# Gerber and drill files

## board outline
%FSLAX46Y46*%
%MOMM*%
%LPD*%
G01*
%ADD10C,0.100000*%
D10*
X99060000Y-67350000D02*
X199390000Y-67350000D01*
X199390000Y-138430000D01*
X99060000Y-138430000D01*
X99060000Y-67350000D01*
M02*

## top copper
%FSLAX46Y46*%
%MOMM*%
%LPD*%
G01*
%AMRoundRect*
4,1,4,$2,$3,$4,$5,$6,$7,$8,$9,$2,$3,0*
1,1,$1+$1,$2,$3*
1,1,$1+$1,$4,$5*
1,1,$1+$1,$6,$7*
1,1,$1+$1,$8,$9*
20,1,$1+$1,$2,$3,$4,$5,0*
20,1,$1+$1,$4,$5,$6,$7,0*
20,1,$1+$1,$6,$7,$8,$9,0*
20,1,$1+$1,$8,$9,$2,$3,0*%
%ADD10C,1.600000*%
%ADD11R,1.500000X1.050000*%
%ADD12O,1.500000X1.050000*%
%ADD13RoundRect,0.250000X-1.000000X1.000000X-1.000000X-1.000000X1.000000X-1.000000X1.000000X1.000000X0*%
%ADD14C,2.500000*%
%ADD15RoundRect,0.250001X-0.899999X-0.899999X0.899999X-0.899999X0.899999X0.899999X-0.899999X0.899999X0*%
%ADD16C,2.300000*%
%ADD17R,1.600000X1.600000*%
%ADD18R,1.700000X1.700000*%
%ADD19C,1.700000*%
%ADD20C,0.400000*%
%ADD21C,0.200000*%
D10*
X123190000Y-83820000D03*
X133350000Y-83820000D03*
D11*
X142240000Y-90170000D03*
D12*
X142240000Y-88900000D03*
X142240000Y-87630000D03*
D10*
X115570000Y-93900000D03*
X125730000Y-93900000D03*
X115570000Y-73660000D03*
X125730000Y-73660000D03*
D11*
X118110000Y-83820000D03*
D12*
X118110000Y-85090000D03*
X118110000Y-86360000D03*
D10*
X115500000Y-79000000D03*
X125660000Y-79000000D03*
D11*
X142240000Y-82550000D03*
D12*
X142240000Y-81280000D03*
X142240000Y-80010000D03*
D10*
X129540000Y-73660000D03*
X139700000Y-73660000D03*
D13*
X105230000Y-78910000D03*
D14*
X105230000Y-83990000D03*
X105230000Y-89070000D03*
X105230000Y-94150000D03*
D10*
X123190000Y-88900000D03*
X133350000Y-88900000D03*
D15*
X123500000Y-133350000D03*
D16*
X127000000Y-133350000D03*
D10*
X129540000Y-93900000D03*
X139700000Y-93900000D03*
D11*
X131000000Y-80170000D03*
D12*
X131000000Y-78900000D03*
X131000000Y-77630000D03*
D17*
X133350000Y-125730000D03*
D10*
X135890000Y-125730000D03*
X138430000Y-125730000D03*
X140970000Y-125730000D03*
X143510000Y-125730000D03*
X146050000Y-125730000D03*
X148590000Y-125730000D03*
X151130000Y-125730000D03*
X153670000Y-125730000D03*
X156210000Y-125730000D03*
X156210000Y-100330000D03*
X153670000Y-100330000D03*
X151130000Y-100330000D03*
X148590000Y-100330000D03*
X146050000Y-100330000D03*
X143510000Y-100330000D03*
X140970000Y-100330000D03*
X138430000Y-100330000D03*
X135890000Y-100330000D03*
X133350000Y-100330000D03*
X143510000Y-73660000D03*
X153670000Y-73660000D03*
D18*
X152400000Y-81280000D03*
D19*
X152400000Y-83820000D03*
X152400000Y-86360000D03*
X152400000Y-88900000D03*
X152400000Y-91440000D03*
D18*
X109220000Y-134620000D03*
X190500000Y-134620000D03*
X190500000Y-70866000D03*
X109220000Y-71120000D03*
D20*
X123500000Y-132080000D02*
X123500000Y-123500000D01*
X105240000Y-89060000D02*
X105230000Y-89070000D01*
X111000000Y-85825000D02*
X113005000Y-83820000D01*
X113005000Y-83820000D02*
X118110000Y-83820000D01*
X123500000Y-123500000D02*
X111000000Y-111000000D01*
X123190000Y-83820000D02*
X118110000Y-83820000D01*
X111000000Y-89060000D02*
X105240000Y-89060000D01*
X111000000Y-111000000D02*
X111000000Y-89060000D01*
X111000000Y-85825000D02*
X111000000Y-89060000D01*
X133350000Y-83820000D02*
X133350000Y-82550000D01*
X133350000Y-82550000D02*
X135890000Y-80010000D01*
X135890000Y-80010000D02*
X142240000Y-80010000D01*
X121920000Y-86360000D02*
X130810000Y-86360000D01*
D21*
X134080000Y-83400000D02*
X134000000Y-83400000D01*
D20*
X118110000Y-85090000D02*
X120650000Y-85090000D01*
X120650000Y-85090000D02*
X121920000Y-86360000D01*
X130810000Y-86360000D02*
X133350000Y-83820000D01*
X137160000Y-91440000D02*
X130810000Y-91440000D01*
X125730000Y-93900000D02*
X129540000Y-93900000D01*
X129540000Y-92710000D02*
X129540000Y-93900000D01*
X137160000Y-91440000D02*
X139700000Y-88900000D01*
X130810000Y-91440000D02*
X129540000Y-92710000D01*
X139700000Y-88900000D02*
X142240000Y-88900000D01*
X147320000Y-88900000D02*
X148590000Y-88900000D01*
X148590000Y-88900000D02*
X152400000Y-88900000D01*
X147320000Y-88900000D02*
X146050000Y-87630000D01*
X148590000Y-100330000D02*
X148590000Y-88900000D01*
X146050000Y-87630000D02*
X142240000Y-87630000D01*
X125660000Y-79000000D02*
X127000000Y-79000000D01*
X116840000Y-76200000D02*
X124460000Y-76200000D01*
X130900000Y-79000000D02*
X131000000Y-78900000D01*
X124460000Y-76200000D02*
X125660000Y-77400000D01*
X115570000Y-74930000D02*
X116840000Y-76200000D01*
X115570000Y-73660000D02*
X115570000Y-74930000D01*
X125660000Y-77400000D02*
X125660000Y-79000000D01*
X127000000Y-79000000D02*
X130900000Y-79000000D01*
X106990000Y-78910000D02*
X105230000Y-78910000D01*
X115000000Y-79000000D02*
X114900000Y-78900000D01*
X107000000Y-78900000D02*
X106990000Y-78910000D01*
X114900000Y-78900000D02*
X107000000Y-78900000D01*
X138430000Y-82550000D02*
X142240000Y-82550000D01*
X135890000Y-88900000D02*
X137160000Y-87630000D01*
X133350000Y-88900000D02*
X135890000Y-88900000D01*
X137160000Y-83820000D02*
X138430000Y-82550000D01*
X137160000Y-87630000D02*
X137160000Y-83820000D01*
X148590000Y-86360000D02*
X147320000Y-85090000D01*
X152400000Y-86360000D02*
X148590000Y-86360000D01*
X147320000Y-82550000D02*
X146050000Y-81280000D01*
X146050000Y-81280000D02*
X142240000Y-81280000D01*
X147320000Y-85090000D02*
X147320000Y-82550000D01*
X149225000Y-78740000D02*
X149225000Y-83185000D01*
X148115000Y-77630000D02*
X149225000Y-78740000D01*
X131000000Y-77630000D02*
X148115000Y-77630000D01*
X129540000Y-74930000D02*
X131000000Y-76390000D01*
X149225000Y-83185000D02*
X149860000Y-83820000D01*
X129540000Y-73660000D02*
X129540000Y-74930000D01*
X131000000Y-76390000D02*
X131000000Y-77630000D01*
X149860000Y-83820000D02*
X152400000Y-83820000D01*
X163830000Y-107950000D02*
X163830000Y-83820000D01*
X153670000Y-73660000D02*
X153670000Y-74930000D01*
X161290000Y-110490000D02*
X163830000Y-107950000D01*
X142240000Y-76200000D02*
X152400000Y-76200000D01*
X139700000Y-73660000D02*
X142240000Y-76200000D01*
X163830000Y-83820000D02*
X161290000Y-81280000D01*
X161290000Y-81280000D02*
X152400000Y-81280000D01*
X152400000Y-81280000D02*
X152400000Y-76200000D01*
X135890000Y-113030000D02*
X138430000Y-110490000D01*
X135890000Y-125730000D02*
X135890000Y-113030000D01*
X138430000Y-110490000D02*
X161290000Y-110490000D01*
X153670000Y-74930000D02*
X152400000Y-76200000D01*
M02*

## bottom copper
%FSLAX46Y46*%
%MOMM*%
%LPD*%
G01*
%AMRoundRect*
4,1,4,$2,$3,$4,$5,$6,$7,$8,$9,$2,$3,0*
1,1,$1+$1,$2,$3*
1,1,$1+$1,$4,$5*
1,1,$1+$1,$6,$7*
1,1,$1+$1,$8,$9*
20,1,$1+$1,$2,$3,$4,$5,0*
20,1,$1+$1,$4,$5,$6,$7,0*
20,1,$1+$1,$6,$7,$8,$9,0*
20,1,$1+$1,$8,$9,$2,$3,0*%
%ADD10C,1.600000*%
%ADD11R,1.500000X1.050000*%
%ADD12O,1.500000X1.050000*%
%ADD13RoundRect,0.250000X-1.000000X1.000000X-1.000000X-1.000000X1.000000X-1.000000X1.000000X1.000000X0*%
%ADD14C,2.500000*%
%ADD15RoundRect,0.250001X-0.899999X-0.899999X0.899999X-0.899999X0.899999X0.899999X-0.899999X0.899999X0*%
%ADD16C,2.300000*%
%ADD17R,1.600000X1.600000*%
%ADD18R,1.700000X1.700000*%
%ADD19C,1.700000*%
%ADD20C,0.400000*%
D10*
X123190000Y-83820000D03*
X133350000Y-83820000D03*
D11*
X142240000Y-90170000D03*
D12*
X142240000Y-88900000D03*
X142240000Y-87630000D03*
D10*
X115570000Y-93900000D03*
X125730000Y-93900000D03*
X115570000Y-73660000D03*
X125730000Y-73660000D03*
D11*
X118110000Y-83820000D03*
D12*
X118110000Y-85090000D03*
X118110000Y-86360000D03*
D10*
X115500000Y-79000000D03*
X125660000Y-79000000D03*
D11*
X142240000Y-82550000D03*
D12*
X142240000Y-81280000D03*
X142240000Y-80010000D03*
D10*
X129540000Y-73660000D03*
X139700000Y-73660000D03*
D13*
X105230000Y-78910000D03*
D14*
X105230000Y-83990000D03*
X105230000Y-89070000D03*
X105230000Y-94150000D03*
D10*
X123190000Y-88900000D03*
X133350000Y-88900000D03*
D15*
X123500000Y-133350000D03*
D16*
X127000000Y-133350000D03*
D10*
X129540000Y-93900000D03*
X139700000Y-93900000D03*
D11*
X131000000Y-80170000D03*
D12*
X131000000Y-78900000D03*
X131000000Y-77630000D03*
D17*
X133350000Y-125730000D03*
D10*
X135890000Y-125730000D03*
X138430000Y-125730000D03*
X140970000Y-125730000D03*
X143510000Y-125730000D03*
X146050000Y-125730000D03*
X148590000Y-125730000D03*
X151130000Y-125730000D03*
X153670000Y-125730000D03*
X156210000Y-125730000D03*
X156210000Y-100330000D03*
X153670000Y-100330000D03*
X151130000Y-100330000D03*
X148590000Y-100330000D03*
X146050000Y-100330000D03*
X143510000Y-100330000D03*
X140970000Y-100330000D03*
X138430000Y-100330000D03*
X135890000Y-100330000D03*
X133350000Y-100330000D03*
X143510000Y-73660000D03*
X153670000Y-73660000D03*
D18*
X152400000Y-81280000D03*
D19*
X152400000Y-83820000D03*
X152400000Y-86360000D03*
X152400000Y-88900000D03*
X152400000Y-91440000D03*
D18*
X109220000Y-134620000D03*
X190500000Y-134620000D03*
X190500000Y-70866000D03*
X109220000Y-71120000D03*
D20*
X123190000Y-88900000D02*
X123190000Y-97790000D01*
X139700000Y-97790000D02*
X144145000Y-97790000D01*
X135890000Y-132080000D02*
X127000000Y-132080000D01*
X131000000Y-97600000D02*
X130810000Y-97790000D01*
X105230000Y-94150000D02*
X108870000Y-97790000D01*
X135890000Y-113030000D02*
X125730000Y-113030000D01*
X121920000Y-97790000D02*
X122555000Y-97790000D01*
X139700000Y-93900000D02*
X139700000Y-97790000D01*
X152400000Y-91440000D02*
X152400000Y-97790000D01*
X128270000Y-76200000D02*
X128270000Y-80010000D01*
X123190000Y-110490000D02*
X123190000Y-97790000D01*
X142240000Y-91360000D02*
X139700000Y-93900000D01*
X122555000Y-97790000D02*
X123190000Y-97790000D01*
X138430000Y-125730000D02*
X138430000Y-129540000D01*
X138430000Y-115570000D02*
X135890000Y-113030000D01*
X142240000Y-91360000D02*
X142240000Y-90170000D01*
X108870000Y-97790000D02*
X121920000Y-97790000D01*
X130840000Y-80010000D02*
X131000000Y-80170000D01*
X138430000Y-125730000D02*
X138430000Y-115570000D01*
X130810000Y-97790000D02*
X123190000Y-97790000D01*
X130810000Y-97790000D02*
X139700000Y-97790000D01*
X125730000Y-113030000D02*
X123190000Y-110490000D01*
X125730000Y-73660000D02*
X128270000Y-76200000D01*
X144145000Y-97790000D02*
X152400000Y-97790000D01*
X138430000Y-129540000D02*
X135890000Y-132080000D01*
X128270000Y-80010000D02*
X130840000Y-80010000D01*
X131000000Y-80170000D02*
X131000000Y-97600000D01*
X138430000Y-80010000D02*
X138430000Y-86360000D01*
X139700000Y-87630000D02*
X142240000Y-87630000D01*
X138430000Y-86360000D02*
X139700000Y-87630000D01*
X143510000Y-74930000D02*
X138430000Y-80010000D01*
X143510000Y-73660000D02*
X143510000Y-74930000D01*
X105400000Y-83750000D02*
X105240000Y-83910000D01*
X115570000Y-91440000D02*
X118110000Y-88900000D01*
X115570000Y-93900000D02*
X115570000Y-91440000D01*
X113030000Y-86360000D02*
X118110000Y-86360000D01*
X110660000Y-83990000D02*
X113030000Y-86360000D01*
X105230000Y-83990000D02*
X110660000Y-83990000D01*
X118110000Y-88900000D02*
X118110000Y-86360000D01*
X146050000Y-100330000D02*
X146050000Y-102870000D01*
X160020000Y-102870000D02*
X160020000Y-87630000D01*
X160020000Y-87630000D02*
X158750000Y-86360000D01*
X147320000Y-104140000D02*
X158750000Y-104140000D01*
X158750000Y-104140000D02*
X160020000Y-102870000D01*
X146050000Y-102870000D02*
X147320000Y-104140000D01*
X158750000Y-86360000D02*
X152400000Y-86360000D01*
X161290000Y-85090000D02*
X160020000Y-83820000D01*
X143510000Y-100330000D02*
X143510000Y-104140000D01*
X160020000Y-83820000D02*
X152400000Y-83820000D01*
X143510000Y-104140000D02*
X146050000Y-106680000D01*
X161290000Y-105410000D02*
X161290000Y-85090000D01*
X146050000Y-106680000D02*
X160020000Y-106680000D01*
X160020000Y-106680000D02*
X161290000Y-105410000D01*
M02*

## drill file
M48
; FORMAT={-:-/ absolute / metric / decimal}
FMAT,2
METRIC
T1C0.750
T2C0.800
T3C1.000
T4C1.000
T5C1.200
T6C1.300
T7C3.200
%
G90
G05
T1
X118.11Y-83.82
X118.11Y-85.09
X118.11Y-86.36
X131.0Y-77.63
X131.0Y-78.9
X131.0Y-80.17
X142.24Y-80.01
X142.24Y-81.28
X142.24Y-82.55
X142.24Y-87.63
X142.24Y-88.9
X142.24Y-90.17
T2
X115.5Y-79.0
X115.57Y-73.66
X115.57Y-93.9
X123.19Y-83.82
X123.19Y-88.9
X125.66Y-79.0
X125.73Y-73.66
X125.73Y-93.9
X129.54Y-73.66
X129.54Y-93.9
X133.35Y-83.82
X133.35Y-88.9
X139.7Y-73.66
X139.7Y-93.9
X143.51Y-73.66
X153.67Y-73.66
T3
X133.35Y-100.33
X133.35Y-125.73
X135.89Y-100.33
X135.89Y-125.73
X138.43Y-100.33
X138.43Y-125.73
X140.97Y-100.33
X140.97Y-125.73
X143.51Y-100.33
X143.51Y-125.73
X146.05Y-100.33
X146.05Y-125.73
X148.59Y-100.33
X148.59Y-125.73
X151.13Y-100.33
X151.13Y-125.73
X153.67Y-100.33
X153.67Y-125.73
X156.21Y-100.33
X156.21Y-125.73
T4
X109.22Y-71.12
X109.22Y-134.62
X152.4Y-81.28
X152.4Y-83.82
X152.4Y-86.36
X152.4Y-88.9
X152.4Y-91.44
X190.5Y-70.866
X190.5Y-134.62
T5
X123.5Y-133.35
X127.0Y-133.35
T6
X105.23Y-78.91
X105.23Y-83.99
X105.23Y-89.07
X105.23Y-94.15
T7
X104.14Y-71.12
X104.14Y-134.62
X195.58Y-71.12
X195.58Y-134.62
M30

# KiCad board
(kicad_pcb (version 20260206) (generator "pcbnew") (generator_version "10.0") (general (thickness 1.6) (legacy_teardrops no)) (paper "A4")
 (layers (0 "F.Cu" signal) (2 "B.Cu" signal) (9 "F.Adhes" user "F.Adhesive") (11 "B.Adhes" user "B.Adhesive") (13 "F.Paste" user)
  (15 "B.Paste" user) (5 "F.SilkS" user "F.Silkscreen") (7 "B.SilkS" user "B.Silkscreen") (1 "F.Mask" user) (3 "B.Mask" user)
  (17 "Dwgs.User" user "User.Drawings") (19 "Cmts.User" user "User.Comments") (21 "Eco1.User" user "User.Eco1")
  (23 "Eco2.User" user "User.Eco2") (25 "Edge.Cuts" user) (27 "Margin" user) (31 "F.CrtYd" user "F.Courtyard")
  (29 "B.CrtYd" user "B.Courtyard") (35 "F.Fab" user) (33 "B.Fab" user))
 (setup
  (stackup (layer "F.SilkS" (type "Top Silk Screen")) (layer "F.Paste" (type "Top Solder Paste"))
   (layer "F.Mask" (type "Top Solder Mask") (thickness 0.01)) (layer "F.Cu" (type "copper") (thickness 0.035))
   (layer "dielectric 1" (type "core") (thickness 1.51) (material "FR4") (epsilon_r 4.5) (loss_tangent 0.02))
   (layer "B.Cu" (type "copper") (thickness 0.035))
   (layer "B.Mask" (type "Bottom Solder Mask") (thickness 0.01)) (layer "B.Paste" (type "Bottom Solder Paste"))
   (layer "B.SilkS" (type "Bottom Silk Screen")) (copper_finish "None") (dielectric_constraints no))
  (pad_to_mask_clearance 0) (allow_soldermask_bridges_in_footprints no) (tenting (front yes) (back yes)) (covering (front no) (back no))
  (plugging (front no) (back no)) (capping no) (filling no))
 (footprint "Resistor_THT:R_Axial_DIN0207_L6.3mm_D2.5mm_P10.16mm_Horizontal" (layer "F.Cu") (at 123.19 83.82)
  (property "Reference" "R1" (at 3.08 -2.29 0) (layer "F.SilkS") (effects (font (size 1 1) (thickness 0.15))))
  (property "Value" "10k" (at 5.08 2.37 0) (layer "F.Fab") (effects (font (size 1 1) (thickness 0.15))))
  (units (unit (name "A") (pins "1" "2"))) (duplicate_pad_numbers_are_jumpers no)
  (pad "1" thru_hole circle (at 0 0) (size 1.6 1.6) (drill 0.8) (layers "*.Cu" "*.Mask") (remove_unused_layers no) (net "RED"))
  (pad "2" thru_hole circle (at 10.16 0) (size 1.6 1.6) (drill 0.8) (layers "*.Cu" "*.Mask") (remove_unused_layers no) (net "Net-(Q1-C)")))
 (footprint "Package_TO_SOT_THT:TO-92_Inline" (layer "F.Cu") (at 142.24 90.17 90)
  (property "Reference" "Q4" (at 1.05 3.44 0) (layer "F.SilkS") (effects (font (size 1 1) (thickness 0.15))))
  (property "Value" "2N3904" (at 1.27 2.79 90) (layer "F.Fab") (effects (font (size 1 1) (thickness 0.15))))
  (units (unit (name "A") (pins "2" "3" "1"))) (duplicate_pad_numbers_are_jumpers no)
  (pad "1" thru_hole rect (at 0 0 90) (size 1.05 1.5) (drill 0.75) (layers "*.Cu" "*.Mask") (remove_unused_layers no) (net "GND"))
  (pad "2" thru_hole oval (at 1.27 0 90) (size 1.05 1.5) (drill 0.75) (layers "*.Cu" "*.Mask") (remove_unused_layers no) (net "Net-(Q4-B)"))
  (pad "3" thru_hole oval (at 2.54 0 90) (size 1.05 1.5) (drill 0.75) (layers "*.Cu" "*.Mask") (remove_unused_layers no) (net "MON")))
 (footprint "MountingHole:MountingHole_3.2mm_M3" (layer "F.Cu") (at 195.58 134.62)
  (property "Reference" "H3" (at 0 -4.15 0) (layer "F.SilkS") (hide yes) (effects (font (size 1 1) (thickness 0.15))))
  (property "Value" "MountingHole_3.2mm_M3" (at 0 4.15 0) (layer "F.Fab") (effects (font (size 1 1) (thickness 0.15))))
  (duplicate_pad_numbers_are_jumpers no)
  (pad "" np_thru_hole circle (at 0 0) (size 3.2 3.2) (drill 3.2) (layers "*.Cu" "*.Mask")))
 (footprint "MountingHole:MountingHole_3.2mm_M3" (layer "F.Cu") (at 104.14 71.12)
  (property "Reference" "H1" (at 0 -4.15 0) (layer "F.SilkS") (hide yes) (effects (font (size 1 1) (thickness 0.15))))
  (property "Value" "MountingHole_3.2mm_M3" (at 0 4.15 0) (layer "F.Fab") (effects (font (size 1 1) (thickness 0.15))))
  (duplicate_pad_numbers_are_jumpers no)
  (pad "" np_thru_hole circle (at 0 0) (size 3.2 3.2) (drill 3.2) (layers "*.Cu" "*.Mask")))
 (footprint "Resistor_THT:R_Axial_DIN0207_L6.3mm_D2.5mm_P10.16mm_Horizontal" (layer "F.Cu") (at 115.57 93.9)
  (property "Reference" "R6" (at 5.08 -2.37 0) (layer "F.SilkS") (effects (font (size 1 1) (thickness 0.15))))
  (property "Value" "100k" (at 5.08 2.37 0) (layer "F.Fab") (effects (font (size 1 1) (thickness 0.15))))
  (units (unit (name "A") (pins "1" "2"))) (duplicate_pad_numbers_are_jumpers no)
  (pad "1" thru_hole circle (at 0 0) (size 1.6 1.6) (drill 0.8) (layers "*.Cu" "*.Mask") (remove_unused_layers no) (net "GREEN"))
  (pad "2" thru_hole circle (at 10.16 0) (size 1.6 1.6) (drill 0.8) (layers "*.Cu" "*.Mask") (remove_unused_layers no) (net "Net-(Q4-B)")))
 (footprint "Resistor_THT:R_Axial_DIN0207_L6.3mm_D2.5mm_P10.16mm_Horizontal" (layer "F.Cu") (at 115.57 73.66)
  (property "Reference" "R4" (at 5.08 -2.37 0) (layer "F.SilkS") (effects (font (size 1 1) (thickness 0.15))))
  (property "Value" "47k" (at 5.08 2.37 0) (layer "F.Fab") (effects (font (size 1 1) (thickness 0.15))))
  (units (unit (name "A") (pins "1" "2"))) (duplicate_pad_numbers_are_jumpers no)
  (pad "1" thru_hole circle (at 0 0) (size 1.6 1.6) (drill 0.8) (layers "*.Cu" "*.Mask") (remove_unused_layers no) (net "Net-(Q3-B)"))
  (pad "2" thru_hole circle (at 10.16 0) (size 1.6 1.6) (drill 0.8) (layers "*.Cu" "*.Mask") (remove_unused_layers no) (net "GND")))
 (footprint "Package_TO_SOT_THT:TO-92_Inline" (layer "F.Cu") (at 118.11 83.82 -90)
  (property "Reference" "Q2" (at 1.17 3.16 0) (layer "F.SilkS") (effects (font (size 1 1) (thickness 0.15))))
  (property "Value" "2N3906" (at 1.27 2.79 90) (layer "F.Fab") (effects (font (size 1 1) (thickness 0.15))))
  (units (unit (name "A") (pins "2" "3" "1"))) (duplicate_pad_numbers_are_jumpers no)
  (pad "1" thru_hole rect (at 0 0 270) (size 1.05 1.5) (drill 0.75) (layers "*.Cu" "*.Mask") (remove_unused_layers no) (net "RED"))
  (pad "2" thru_hole oval (at 1.27 0 270) (size 1.05 1.5) (drill 0.75) (layers "*.Cu" "*.Mask") (remove_unused_layers no) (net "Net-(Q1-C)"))
  (pad "3" thru_hole oval (at 2.54 0 270) (size 1.05 1.5) (drill 0.75) (layers "*.Cu" "*.Mask") (remove_unused_layers no) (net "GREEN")))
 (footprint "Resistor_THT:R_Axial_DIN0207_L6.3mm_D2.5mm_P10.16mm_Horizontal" (layer "F.Cu") (at 115.5 79)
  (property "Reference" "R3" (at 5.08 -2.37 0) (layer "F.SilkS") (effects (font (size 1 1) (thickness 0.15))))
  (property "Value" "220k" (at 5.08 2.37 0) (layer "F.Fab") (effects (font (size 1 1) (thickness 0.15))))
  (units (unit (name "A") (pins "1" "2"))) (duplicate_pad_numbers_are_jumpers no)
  (pad "1" thru_hole circle (at 0 0) (size 1.6 1.6) (drill 0.8) (layers "*.Cu" "*.Mask") (remove_unused_layers no) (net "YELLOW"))
  (pad "2" thru_hole circle (at 10.16 0) (size 1.6 1.6) (drill 0.8) (layers "*.Cu" "*.Mask") (remove_unused_layers no) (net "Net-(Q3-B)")))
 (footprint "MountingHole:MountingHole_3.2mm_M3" (layer "F.Cu") (at 195.58 71.12)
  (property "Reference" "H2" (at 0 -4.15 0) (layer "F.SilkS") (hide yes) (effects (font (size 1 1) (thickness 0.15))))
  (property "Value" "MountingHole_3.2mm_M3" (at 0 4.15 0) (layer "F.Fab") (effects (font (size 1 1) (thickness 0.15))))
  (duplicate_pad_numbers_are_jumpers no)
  (pad "" np_thru_hole circle (at 0 0) (size 3.2 3.2) (drill 3.2) (layers "*.Cu" "*.Mask")))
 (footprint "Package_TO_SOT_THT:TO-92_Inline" (layer "F.Cu") (at 142.24 82.55 90)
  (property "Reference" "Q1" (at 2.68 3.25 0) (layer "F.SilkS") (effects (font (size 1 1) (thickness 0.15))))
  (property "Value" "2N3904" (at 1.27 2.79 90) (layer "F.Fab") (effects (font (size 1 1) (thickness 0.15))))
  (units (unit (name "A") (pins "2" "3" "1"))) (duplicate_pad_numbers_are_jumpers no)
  (pad "1" thru_hole rect (at 0 0 90) (size 1.05 1.5) (drill 0.75) (layers "*.Cu" "*.Mask") (remove_unused_layers no) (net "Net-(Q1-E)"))
  (pad "2" thru_hole oval (at 1.27 0 90) (size 1.05 1.5) (drill 0.75) (layers "*.Cu" "*.Mask") (remove_unused_layers no) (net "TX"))
  (pad "3" thru_hole oval (at 2.54 0 90) (size 1.05 1.5) (drill 0.75) (layers "*.Cu" "*.Mask") (remove_unused_layers no) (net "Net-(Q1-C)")))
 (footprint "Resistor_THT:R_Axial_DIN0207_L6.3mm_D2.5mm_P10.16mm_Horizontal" (layer "F.Cu") (at 129.54 73.66)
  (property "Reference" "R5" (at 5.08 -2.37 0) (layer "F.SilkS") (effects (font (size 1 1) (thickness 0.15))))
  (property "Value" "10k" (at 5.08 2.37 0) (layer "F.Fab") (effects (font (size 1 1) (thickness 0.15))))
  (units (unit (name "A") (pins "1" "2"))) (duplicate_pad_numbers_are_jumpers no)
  (pad "1" thru_hole circle (at 0 0) (size 1.6 1.6) (drill 0.8) (layers "*.Cu" "*.Mask") (remove_unused_layers no) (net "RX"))
  (pad "2" thru_hole circle (at 10.16 0) (size 1.6 1.6) (drill 0.8) (layers "*.Cu" "*.Mask") (remove_unused_layers no) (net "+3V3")))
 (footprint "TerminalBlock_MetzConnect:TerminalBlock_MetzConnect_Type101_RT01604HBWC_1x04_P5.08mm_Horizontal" (layer "F.Cu")
  (at 105.23 78.91 -90)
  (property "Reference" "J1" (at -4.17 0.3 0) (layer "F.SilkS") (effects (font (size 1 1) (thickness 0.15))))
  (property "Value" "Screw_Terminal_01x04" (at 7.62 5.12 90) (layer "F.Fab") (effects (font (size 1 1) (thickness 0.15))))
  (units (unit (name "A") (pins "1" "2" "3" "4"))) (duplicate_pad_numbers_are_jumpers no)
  (pad "1" thru_hole roundrect (at 0 0 270) (size 2.5 2.5) (drill 1.3) (layers "*.Cu" "*.Mask") (remove_unused_layers no)
   (roundrect_rratio 0.1) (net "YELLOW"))
  (pad "2" thru_hole circle (at 5.08 0 270) (size 2.5 2.5) (drill 1.3) (layers "*.Cu" "*.Mask") (remove_unused_layers no) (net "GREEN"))
  (pad "3" thru_hole circle (at 10.16 0 270) (size 2.5 2.5) (drill 1.3) (layers "*.Cu" "*.Mask") (remove_unused_layers no) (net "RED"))
  (pad "4" thru_hole circle (at 15.24 0 270) (size 2.5 2.5) (drill 1.3) (layers "*.Cu" "*.Mask") (remove_unused_layers no) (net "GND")))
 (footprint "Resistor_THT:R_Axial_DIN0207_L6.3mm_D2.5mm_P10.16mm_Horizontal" (layer "F.Cu") (at 123.19 88.9)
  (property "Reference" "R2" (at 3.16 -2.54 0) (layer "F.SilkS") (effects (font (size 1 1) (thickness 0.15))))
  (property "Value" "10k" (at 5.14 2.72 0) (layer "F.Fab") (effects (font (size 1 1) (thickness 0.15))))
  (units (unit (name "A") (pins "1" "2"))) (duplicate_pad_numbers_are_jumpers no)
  (pad "1" thru_hole circle (at 0 0) (size 1.6 1.6) (drill 0.8) (layers "*.Cu" "*.Mask") (remove_unused_layers no) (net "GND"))
  (pad "2" thru_hole circle (at 10.16 0) (size 1.6 1.6) (drill 0.8) (layers "*.Cu" "*.Mask") (remove_unused_layers no) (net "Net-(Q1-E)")))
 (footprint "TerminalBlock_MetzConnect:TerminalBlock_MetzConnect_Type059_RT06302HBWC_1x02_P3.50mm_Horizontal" (layer "F.Cu")
  (at 123.5 133.35)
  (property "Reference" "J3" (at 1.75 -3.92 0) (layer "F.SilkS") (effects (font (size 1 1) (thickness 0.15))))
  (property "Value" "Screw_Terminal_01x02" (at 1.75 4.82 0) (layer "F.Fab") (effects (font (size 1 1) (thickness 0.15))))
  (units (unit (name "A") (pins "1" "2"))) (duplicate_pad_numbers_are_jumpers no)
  (pad "1" thru_hole roundrect (at 0 0) (size 2.3 2.3) (drill 1.2) (layers "*.Cu" "*.Mask") (remove_unused_layers no)
   (roundrect_rratio 0.108696) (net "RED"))
  (pad "2" thru_hole circle (at 3.5 0) (size 2.3 2.3) (drill 1.2) (layers "*.Cu" "*.Mask") (remove_unused_layers no) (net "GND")))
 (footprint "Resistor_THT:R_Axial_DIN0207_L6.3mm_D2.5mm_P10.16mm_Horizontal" (layer "F.Cu") (at 129.54 93.9)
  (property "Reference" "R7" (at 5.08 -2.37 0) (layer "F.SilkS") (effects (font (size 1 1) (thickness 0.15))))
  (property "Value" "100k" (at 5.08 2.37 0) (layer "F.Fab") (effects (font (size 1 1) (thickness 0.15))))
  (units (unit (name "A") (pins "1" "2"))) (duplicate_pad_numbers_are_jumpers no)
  (pad "1" thru_hole circle (at 0 0) (size 1.6 1.6) (drill 0.8) (layers "*.Cu" "*.Mask") (remove_unused_layers no) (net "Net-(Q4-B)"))
  (pad "2" thru_hole circle (at 10.16 0) (size 1.6 1.6) (drill 0.8) (layers "*.Cu" "*.Mask") (remove_unused_layers no) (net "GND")))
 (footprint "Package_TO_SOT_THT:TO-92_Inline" (layer "F.Cu") (at 131 80.17 90)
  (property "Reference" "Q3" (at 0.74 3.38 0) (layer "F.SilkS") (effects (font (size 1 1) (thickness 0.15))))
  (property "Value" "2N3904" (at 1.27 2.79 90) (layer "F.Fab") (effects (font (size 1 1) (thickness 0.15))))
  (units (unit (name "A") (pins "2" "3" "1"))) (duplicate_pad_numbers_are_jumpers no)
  (pad "1" thru_hole rect (at 0 0 90) (size 1.05 1.5) (drill 0.75) (layers "*.Cu" "*.Mask") (remove_unused_layers no) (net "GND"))
  (pad "2" thru_hole oval (at 1.27 0 90) (size 1.05 1.5) (drill 0.75) (layers "*.Cu" "*.Mask") (remove_unused_layers no) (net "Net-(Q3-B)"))
  (pad "3" thru_hole oval (at 2.54 0 90) (size 1.05 1.5) (drill 0.75) (layers "*.Cu" "*.Mask") (remove_unused_layers no) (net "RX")))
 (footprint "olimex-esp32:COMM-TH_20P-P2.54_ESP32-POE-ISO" (layer "F.Cu") (at 144.78 113.03 90)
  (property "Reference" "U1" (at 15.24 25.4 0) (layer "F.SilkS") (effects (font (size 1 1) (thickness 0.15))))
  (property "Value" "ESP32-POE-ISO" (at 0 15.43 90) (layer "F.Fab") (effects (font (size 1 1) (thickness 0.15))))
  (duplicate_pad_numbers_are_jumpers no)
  (pad "1" thru_hole rect (at -12.7 -11.43 90) (size 1.6 1.6) (drill 0.999998) (layers "*.Cu" "*.Mask") (remove_unused_layers no)
   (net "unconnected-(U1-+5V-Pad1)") (thermal_bridge_angle 45))
  (pad "2" thru_hole circle (at -12.7 -8.89 90) (size 1.6 1.6) (drill 0.999998) (layers "*.Cu" "*.Mask") (remove_unused_layers no)
   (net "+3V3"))
  (pad "3" thru_hole circle (at -12.7 -6.35 90) (size 1.6 1.6) (drill 0.999998) (layers "*.Cu" "*.Mask") (remove_unused_layers no)
   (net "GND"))
  (pad "4" thru_hole circle (at -12.7 -3.81 90) (size 1.6 1.6) (drill 0.999998) (layers "*.Cu" "*.Mask") (remove_unused_layers no)
   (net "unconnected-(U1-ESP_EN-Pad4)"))
  (pad "5" thru_hole circle (at -12.7 -1.27 90) (size 1.6 1.6) (drill 0.999998) (layers "*.Cu" "*.Mask") (remove_unused_layers no)
   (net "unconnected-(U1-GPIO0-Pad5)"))
  (pad "6" thru_hole circle (at -12.7 1.27 90) (size 1.6 1.6) (drill 0.999998) (layers "*.Cu" "*.Mask") (remove_unused_layers no)
   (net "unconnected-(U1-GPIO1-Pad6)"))
  (pad "7" thru_hole circle (at -12.7 3.81 90) (size 1.6 1.6) (drill 0.999998) (layers "*.Cu" "*.Mask") (remove_unused_layers no)
   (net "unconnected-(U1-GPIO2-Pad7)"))
  (pad "8" thru_hole circle (at -12.7 6.35 90) (size 1.6 1.6) (drill 0.999998) (layers "*.Cu" "*.Mask") (remove_unused_layers no)
   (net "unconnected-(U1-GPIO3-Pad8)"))
  (pad "9" thru_hole circle (at -12.7 8.89 90) (size 1.6 1.6) (drill 0.999998) (layers "*.Cu" "*.Mask") (remove_unused_layers no)
   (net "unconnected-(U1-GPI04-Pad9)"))
  (pad "10" thru_hole circle (at -12.7 11.43 90) (size 1.6 1.6) (drill 0.999998) (layers "*.Cu" "*.Mask") (remove_unused_layers no)
   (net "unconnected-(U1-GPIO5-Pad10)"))
  (pad "11" thru_hole circle (at 12.7 11.43 90) (size 1.6 1.6) (drill 0.999998) (layers "*.Cu" "*.Mask") (remove_unused_layers no)
   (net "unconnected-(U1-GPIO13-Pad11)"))
  (pad "12" thru_hole circle (at 12.7 8.89 90) (size 1.6 1.6) (drill 0.999998) (layers "*.Cu" "*.Mask") (remove_unused_layers no)
   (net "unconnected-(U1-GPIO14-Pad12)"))
  (pad "13" thru_hole circle (at 12.7 6.35 90) (size 1.6 1.6) (drill 0.999998) (layers "*.Cu" "*.Mask") (remove_unused_layers no)
   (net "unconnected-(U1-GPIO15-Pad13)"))
  (pad "14" thru_hole circle (at 12.7 3.81 90) (size 1.6 1.6) (drill 0.999998) (layers "*.Cu" "*.Mask") (remove_unused_layers no)
   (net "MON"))
  (pad "15" thru_hole circle (at 12.7 1.27 90) (size 1.6 1.6) (drill 0.999998) (layers "*.Cu" "*.Mask") (remove_unused_layers no) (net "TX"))
  (pad "16" thru_hole circle (at 12.7 -1.27 90) (size 1.6 1.6) (drill 0.999998) (layers "*.Cu" "*.Mask") (remove_unused_layers no)
   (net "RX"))
  (pad "17" thru_hole circle (at 12.7 -3.81 90) (size 1.6 1.6) (drill 0.999998) (layers "*.Cu" "*.Mask") (remove_unused_layers no)
   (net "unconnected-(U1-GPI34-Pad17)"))
  (pad "18" thru_hole circle (at 12.7 -6.35 90) (size 1.6 1.6) (drill 0.999998) (layers "*.Cu" "*.Mask") (remove_unused_layers no)
   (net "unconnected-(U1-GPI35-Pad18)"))
  (pad "19" thru_hole circle (at 12.7 -8.89 90) (size 1.6 1.6) (drill 0.999998) (layers "*.Cu" "*.Mask") (remove_unused_layers no)
   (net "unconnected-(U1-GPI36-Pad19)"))
  (pad "20" thru_hole circle (at 12.7 -11.43 90) (size 1.6 1.6) (drill 0.999998) (layers "*.Cu" "*.Mask") (remove_unused_layers no)
   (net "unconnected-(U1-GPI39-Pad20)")))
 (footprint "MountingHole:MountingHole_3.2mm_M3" (layer "F.Cu") (at 104.14 134.62)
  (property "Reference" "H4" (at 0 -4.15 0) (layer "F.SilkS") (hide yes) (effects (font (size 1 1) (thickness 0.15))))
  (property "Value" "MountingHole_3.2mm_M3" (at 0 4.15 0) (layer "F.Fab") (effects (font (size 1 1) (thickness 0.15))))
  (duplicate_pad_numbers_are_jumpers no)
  (pad "" np_thru_hole circle (at 0 0) (size 3.2 3.2) (drill 3.2) (layers "*.Cu" "*.Mask")))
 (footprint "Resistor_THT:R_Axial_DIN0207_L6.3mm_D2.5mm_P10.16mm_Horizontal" (layer "F.Cu") (at 143.51 73.66)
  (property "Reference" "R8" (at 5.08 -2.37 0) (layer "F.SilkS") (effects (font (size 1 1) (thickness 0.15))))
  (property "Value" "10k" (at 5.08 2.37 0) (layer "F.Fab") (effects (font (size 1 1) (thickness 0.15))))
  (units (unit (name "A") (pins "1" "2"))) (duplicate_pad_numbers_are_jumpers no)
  (pad "1" thru_hole circle (at 0 0) (size 1.6 1.6) (drill 0.8) (layers "*.Cu" "*.Mask") (remove_unused_layers no) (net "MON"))
  (pad "2" thru_hole circle (at 10.16 0) (size 1.6 1.6) (drill 0.8) (layers "*.Cu" "*.Mask") (remove_unused_layers no) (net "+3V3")))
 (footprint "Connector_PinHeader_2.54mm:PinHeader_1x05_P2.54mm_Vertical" (layer "F.Cu") (at 152.4 81.28)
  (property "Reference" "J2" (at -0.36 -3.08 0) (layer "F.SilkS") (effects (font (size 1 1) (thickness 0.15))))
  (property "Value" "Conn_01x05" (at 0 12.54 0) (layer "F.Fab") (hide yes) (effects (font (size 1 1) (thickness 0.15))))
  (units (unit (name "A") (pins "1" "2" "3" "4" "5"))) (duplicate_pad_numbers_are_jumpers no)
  (pad "1" thru_hole rect (at 0 0) (size 1.7 1.7) (drill 1) (layers "*.Cu" "*.Mask") (remove_unused_layers no) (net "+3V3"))
  (pad "2" thru_hole circle (at 0 2.54) (size 1.7 1.7) (drill 1) (layers "*.Cu" "*.Mask") (remove_unused_layers no) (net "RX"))
  (pad "3" thru_hole circle (at 0 5.08) (size 1.7 1.7) (drill 1) (layers "*.Cu" "*.Mask") (remove_unused_layers no) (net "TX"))
  (pad "4" thru_hole circle (at 0 7.62) (size 1.7 1.7) (drill 1) (layers "*.Cu" "*.Mask") (remove_unused_layers no) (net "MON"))
  (pad "5" thru_hole circle (at 0 10.16) (size 1.7 1.7) (drill 1) (layers "*.Cu" "*.Mask") (remove_unused_layers no) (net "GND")))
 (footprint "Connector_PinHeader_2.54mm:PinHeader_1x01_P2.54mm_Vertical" (layer "B.Cu") (at 109.22 134.62)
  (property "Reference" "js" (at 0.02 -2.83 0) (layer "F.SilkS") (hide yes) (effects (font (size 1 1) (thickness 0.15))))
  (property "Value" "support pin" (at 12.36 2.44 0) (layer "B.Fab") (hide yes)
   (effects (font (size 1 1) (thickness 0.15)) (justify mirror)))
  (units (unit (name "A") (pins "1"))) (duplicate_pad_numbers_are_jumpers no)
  (pad "1" thru_hole rect (at 0 0) (size 1.7 1.7) (drill 1) (layers "*.Cu" "*.Mask") (remove_unused_layers no)
   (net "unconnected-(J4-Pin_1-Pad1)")))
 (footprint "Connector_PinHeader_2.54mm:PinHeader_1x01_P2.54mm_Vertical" (layer "B.Cu") (at 190.5 134.62)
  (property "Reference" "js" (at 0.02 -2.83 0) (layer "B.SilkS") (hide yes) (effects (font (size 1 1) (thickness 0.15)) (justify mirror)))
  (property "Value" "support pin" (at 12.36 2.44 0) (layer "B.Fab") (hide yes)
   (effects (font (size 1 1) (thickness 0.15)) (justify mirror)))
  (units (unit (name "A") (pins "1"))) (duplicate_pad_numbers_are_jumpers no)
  (pad "1" thru_hole rect (at 0 0) (size 1.7 1.7) (drill 1) (layers "*.Cu" "*.Mask") (remove_unused_layers no)
   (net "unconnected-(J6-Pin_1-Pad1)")))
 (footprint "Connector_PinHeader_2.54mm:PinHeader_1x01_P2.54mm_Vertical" (layer "B.Cu") (at 190.5 70.866)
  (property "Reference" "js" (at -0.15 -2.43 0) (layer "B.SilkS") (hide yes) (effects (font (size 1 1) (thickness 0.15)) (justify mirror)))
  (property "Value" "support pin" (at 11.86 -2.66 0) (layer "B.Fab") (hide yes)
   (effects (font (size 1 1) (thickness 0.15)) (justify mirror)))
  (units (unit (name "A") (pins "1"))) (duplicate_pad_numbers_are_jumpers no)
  (pad "1" thru_hole rect (at 0 0) (size 1.7 1.7) (drill 1) (layers "*.Cu" "*.Mask") (remove_unused_layers no)
   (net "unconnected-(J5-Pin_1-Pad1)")))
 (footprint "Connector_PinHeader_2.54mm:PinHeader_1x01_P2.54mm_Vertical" (layer "B.Cu") (at 109.22 71.12)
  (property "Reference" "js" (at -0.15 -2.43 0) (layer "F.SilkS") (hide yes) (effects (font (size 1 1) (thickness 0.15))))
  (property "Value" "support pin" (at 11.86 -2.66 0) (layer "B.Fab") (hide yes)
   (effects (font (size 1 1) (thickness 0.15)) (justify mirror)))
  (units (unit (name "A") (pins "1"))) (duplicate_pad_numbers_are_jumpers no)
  (pad "1" thru_hole rect (at 0 0) (size 1.7 1.7) (drill 1) (layers "*.Cu" "*.Mask") (remove_unused_layers no)
   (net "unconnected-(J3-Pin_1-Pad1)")))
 (gr_rect (start 99.06 67.35) (end 199.39 138.43) (stroke (width 0.1) (type default)) (fill no) (layer "Edge.Cuts"))
 (segment (start 123.5 132.08) (end 123.5 123.5) (width 0.4) (layer "F.Cu") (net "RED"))
 (segment (start 105.24 89.06) (end 105.23 89.07) (width 0.4) (layer "F.Cu") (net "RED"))
 (segment (start 111 85.825) (end 113.005 83.82) (width 0.4) (layer "F.Cu") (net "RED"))
 (segment (start 113.005 83.82) (end 118.11 83.82) (width 0.4) (layer "F.Cu") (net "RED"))
 (segment (start 123.5 123.5) (end 111 111) (width 0.4) (layer "F.Cu") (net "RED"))
 (segment (start 123.19 83.82) (end 118.11 83.82) (width 0.4) (layer "F.Cu") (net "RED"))
 (segment (start 111 89.06) (end 105.24 89.06) (width 0.4) (layer "F.Cu") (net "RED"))
 (segment (start 111 111) (end 111 89.06) (width 0.4) (layer "F.Cu") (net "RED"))
 (segment (start 111 85.825) (end 111 89.06) (width 0.4) (layer "F.Cu") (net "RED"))
 (segment (start 133.35 83.82) (end 133.35 82.55) (width 0.4) (layer "F.Cu") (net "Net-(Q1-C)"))
 (segment (start 133.35 82.55) (end 135.89 80.01) (width 0.4) (layer "F.Cu") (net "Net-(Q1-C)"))
 (segment (start 135.89 80.01) (end 142.24 80.01) (width 0.4) (layer "F.Cu") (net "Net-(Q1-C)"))
 (segment (start 121.92 86.36) (end 130.81 86.36) (width 0.4) (layer "F.Cu") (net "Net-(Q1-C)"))
 (segment (start 134.08 83.4) (end 134 83.4) (width 0.2) (layer "F.Cu") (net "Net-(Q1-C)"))
 (segment (start 118.11 85.09) (end 120.65 85.09) (width 0.4) (layer "F.Cu") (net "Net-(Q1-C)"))
 (segment (start 120.65 85.09) (end 121.92 86.36) (width 0.4) (layer "F.Cu") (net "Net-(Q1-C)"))
 (segment (start 130.81 86.36) (end 133.35 83.82) (width 0.4) (layer "F.Cu") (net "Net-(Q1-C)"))
 (segment (start 123.19 88.9) (end 123.19 97.79) (width 0.4) (layer "B.Cu") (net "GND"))
 (segment (start 139.7 97.79) (end 144.145 97.79) (width 0.4) (layer "B.Cu") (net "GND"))
 (segment (start 135.89 132.08) (end 127 132.08) (width 0.4) (layer "B.Cu") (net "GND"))
 (segment (start 131 97.6) (end 130.81 97.79) (width 0.4) (layer "B.Cu") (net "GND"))
 (segment (start 105.23 94.15) (end 108.87 97.79) (width 0.4) (layer "B.Cu") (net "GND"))
 (segment (start 135.89 113.03) (end 125.73 113.03) (width 0.4) (layer "B.Cu") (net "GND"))
 (segment (start 121.92 97.79) (end 122.555 97.79) (width 0.4) (layer "B.Cu") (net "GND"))
 (segment (start 139.7 93.9) (end 139.7 97.79) (width 0.4) (layer "B.Cu") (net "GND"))
 (segment (start 152.4 91.44) (end 152.4 97.79) (width 0.4) (layer "B.Cu") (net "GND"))
 (segment (start 128.27 76.2) (end 128.27 80.01) (width 0.4) (layer "B.Cu") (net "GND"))
 (segment (start 123.19 110.49) (end 123.19 97.79) (width 0.4) (layer "B.Cu") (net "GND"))
 (segment (start 142.24 91.36) (end 139.7 93.9) (width 0.4) (layer "B.Cu") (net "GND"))
 (segment (start 122.555 97.79) (end 123.19 97.79) (width 0.4) (layer "B.Cu") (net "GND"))
 (segment (start 138.43 125.73) (end 138.43 129.54) (width 0.4) (layer "B.Cu") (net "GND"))
 (segment (start 138.43 115.57) (end 135.89 113.03) (width 0.4) (layer "B.Cu") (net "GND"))
 (segment (start 142.24 91.36) (end 142.24 90.17) (width 0.4) (layer "B.Cu") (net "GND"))
 (segment (start 108.87 97.79) (end 121.92 97.79) (width 0.4) (layer "B.Cu") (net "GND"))
 (segment (start 130.84 80.01) (end 131 80.17) (width 0.4) (layer "B.Cu") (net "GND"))
 (segment (start 138.43 125.73) (end 138.43 115.57) (width 0.4) (layer "B.Cu") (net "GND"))
 (segment (start 130.81 97.79) (end 123.19 97.79) (width 0.4) (layer "B.Cu") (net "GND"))
 (segment (start 130.81 97.79) (end 139.7 97.79) (width 0.4) (layer "B.Cu") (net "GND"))
 (segment (start 125.73 113.03) (end 123.19 110.49) (width 0.4) (layer "B.Cu") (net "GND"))
 (segment (start 125.73 73.66) (end 128.27 76.2) (width 0.4) (layer "B.Cu") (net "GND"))
 (segment (start 144.145 97.79) (end 152.4 97.79) (width 0.4) (layer "B.Cu") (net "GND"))
 (segment (start 138.43 129.54) (end 135.89 132.08) (width 0.4) (layer "B.Cu") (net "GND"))
 (segment (start 128.27 80.01) (end 130.84 80.01) (width 0.4) (layer "B.Cu") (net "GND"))
 (segment (start 131 80.17) (end 131 97.6) (width 0.4) (layer "B.Cu") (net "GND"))
 (segment (start 137.16 91.44) (end 130.81 91.44) (width 0.4) (layer "F.Cu") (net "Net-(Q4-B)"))
 (segment (start 125.73 93.9) (end 129.54 93.9) (width 0.4) (layer "F.Cu") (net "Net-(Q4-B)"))
 (segment (start 129.54 92.71) (end 129.54 93.9) (width 0.4) (layer "F.Cu") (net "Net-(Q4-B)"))
 (segment (start 137.16 91.44) (end 139.7 88.9) (width 0.4) (layer "F.Cu") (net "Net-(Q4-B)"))
 (segment (start 130.81 91.44) (end 129.54 92.71) (width 0.4) (layer "F.Cu") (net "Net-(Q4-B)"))
 (segment (start 139.7 88.9) (end 142.24 88.9) (width 0.4) (layer "F.Cu") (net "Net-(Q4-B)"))
 (segment (start 147.32 88.9) (end 148.59 88.9) (width 0.4) (layer "F.Cu") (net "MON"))
 (segment (start 148.59 88.9) (end 152.4 88.9) (width 0.4) (layer "F.Cu") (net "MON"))
 (segment (start 147.32 88.9) (end 146.05 87.63) (width 0.4) (layer "F.Cu") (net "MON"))
 (segment (start 148.59 100.33) (end 148.59 88.9) (width 0.4) (layer "F.Cu") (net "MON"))
 (segment (start 146.05 87.63) (end 142.24 87.63) (width 0.4) (layer "F.Cu") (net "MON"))
 (segment (start 138.43 80.01) (end 138.43 86.36) (width 0.4) (layer "B.Cu") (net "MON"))
 (segment (start 139.7 87.63) (end 142.24 87.63) (width 0.4) (layer "B.Cu") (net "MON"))
 (segment (start 138.43 86.36) (end 139.7 87.63) (width 0.4) (layer "B.Cu") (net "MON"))
 (segment (start 143.51 74.93) (end 138.43 80.01) (width 0.4) (layer "B.Cu") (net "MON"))
 (segment (start 143.51 73.66) (end 143.51 74.93) (width 0.4) (layer "B.Cu") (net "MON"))
 (segment (start 105.4 83.75) (end 105.24 83.91) (width 0.4) (layer "B.Cu") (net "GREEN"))
 (segment (start 115.57 91.44) (end 118.11 88.9) (width 0.4) (layer "B.Cu") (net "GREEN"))
 (segment (start 115.57 93.9) (end 115.57 91.44) (width 0.4) (layer "B.Cu") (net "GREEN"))
 (segment (start 113.03 86.36) (end 118.11 86.36) (width 0.4) (layer "B.Cu") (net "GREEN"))
 (segment (start 110.66 83.99) (end 113.03 86.36) (width 0.4) (layer "B.Cu") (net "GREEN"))
 (segment (start 105.23 83.99) (end 110.66 83.99) (width 0.4) (layer "B.Cu") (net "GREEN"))
 (segment (start 118.11 88.9) (end 118.11 86.36) (width 0.4) (layer "B.Cu") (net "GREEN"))
 (segment (start 125.66 79) (end 127 79) (width 0.4) (layer "F.Cu") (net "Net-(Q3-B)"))
 (segment (start 116.84 76.2) (end 124.46 76.2) (width 0.4) (layer "F.Cu") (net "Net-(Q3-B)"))
 (segment (start 130.9 79) (end 131 78.9) (width 0.4) (layer "F.Cu") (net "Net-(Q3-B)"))
 (segment (start 124.46 76.2) (end 125.66 77.4) (width 0.4) (layer "F.Cu") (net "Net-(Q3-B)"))
 (segment (start 115.57 74.93) (end 116.84 76.2) (width 0.4) (layer "F.Cu") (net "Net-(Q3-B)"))
 (segment (start 115.57 73.66) (end 115.57 74.93) (width 0.4) (layer "F.Cu") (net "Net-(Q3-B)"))
 (segment (start 125.66 77.4) (end 125.66 79) (width 0.4) (layer "F.Cu") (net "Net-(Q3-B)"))
 (segment (start 127 79) (end 130.9 79) (width 0.4) (layer "F.Cu") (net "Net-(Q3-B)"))
 (segment (start 106.99 78.91) (end 105.23 78.91) (width 0.4) (layer "F.Cu") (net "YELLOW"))
 (segment (start 115 79) (end 114.9 78.9) (width 0.4) (layer "F.Cu") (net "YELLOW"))
 (segment (start 107 78.9) (end 106.99 78.91) (width 0.4) (layer "F.Cu") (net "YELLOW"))
 (segment (start 114.9 78.9) (end 107 78.9) (width 0.4) (layer "F.Cu") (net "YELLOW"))
 (segment (start 138.43 82.55) (end 142.24 82.55) (width 0.4) (layer "F.Cu") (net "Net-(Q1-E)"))
 (segment (start 135.89 88.9) (end 137.16 87.63) (width 0.4) (layer "F.Cu") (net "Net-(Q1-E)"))
 (segment (start 133.35 88.9) (end 135.89 88.9) (width 0.4) (layer "F.Cu") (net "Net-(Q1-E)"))
 (segment (start 137.16 83.82) (end 138.43 82.55) (width 0.4) (layer "F.Cu") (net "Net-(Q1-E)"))
 (segment (start 137.16 87.63) (end 137.16 83.82) (width 0.4) (layer "F.Cu") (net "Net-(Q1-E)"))
 (segment (start 148.59 86.36) (end 147.32 85.09) (width 0.4) (layer "F.Cu") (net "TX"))
 (segment (start 152.4 86.36) (end 148.59 86.36) (width 0.4) (layer "F.Cu") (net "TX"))
 (segment (start 147.32 82.55) (end 146.05 81.28) (width 0.4) (layer "F.Cu") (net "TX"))
 (segment (start 146.05 81.28) (end 142.24 81.28) (width 0.4) (layer "F.Cu") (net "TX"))
 (segment (start 147.32 85.09) (end 147.32 82.55) (width 0.4) (layer "F.Cu") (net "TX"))
 (segment (start 146.05 100.33) (end 146.05 102.87) (width 0.4) (layer "B.Cu") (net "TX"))
 (segment (start 160.02 102.87) (end 160.02 87.63) (width 0.4) (layer "B.Cu") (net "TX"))
 (segment (start 160.02 87.63) (end 158.75 86.36) (width 0.4) (layer "B.Cu") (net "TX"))
 (segment (start 147.32 104.14) (end 158.75 104.14) (width 0.4) (layer "B.Cu") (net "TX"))
 (segment (start 158.75 104.14) (end 160.02 102.87) (width 0.4) (layer "B.Cu") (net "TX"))
 (segment (start 146.05 102.87) (end 147.32 104.14) (width 0.4) (layer "B.Cu") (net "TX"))
 (segment (start 158.75 86.36) (end 152.4 86.36) (width 0.4) (layer "B.Cu") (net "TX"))
 (segment (start 149.225 78.74) (end 149.225 83.185) (width 0.4) (layer "F.Cu") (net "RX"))
 (segment (start 148.115 77.63) (end 149.225 78.74) (width 0.4) (layer "F.Cu") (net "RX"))
 (segment (start 131 77.63) (end 148.115 77.63) (width 0.4) (layer "F.Cu") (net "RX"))
 (segment (start 129.54 74.93) (end 131 76.39) (width 0.4) (layer "F.Cu") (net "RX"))
 (segment (start 149.225 83.185) (end 149.86 83.82) (width 0.4) (layer "F.Cu") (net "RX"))
 (segment (start 129.54 73.66) (end 129.54 74.93) (width 0.4) (layer "F.Cu") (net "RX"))
 (segment (start 131 76.39) (end 131 77.63) (width 0.4) (layer "F.Cu") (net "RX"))
 (segment (start 149.86 83.82) (end 152.4 83.82) (width 0.4) (layer "F.Cu") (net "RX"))
 (segment (start 161.29 85.09) (end 160.02 83.82) (width 0.4) (layer "B.Cu") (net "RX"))
 (segment (start 143.51 100.33) (end 143.51 104.14) (width 0.4) (layer "B.Cu") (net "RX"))
 (segment (start 160.02 83.82) (end 152.4 83.82) (width 0.4) (layer "B.Cu") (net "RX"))
 (segment (start 143.51 104.14) (end 146.05 106.68) (width 0.4) (layer "B.Cu") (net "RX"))
 (segment (start 161.29 105.41) (end 161.29 85.09) (width 0.4) (layer "B.Cu") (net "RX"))
 (segment (start 146.05 106.68) (end 160.02 106.68) (width 0.4) (layer "B.Cu") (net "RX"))
 (segment (start 160.02 106.68) (end 161.29 105.41) (width 0.4) (layer "B.Cu") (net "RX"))
 (segment (start 163.83 107.95) (end 163.83 83.82) (width 0.4) (layer "F.Cu") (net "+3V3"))
 (segment (start 153.67 73.66) (end 153.67 74.93) (width 0.4) (layer "F.Cu") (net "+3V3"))
 (segment (start 161.29 110.49) (end 163.83 107.95) (width 0.4) (layer "F.Cu") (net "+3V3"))
 (segment (start 142.24 76.2) (end 152.4 76.2) (width 0.4) (layer "F.Cu") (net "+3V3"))
 (segment (start 139.7 73.66) (end 142.24 76.2) (width 0.4) (layer "F.Cu") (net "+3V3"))
 (segment (start 163.83 83.82) (end 161.29 81.28) (width 0.4) (layer "F.Cu") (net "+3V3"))
 (segment (start 161.29 81.28) (end 152.4 81.28) (width 0.4) (layer "F.Cu") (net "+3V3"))
 (segment (start 152.4 81.28) (end 152.4 76.2) (width 0.4) (layer "F.Cu") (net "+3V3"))
 (segment (start 135.89 113.03) (end 138.43 110.49) (width 0.4) (layer "F.Cu") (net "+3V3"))
 (segment (start 135.89 125.73) (end 135.89 113.03) (width 0.4) (layer "F.Cu") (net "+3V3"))
 (segment (start 138.43 110.49) (end 161.29 110.49) (width 0.4) (layer "F.Cu") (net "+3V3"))
 (segment (start 153.67 74.93) (end 152.4 76.2) (width 0.4) (layer "F.Cu") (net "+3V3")))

